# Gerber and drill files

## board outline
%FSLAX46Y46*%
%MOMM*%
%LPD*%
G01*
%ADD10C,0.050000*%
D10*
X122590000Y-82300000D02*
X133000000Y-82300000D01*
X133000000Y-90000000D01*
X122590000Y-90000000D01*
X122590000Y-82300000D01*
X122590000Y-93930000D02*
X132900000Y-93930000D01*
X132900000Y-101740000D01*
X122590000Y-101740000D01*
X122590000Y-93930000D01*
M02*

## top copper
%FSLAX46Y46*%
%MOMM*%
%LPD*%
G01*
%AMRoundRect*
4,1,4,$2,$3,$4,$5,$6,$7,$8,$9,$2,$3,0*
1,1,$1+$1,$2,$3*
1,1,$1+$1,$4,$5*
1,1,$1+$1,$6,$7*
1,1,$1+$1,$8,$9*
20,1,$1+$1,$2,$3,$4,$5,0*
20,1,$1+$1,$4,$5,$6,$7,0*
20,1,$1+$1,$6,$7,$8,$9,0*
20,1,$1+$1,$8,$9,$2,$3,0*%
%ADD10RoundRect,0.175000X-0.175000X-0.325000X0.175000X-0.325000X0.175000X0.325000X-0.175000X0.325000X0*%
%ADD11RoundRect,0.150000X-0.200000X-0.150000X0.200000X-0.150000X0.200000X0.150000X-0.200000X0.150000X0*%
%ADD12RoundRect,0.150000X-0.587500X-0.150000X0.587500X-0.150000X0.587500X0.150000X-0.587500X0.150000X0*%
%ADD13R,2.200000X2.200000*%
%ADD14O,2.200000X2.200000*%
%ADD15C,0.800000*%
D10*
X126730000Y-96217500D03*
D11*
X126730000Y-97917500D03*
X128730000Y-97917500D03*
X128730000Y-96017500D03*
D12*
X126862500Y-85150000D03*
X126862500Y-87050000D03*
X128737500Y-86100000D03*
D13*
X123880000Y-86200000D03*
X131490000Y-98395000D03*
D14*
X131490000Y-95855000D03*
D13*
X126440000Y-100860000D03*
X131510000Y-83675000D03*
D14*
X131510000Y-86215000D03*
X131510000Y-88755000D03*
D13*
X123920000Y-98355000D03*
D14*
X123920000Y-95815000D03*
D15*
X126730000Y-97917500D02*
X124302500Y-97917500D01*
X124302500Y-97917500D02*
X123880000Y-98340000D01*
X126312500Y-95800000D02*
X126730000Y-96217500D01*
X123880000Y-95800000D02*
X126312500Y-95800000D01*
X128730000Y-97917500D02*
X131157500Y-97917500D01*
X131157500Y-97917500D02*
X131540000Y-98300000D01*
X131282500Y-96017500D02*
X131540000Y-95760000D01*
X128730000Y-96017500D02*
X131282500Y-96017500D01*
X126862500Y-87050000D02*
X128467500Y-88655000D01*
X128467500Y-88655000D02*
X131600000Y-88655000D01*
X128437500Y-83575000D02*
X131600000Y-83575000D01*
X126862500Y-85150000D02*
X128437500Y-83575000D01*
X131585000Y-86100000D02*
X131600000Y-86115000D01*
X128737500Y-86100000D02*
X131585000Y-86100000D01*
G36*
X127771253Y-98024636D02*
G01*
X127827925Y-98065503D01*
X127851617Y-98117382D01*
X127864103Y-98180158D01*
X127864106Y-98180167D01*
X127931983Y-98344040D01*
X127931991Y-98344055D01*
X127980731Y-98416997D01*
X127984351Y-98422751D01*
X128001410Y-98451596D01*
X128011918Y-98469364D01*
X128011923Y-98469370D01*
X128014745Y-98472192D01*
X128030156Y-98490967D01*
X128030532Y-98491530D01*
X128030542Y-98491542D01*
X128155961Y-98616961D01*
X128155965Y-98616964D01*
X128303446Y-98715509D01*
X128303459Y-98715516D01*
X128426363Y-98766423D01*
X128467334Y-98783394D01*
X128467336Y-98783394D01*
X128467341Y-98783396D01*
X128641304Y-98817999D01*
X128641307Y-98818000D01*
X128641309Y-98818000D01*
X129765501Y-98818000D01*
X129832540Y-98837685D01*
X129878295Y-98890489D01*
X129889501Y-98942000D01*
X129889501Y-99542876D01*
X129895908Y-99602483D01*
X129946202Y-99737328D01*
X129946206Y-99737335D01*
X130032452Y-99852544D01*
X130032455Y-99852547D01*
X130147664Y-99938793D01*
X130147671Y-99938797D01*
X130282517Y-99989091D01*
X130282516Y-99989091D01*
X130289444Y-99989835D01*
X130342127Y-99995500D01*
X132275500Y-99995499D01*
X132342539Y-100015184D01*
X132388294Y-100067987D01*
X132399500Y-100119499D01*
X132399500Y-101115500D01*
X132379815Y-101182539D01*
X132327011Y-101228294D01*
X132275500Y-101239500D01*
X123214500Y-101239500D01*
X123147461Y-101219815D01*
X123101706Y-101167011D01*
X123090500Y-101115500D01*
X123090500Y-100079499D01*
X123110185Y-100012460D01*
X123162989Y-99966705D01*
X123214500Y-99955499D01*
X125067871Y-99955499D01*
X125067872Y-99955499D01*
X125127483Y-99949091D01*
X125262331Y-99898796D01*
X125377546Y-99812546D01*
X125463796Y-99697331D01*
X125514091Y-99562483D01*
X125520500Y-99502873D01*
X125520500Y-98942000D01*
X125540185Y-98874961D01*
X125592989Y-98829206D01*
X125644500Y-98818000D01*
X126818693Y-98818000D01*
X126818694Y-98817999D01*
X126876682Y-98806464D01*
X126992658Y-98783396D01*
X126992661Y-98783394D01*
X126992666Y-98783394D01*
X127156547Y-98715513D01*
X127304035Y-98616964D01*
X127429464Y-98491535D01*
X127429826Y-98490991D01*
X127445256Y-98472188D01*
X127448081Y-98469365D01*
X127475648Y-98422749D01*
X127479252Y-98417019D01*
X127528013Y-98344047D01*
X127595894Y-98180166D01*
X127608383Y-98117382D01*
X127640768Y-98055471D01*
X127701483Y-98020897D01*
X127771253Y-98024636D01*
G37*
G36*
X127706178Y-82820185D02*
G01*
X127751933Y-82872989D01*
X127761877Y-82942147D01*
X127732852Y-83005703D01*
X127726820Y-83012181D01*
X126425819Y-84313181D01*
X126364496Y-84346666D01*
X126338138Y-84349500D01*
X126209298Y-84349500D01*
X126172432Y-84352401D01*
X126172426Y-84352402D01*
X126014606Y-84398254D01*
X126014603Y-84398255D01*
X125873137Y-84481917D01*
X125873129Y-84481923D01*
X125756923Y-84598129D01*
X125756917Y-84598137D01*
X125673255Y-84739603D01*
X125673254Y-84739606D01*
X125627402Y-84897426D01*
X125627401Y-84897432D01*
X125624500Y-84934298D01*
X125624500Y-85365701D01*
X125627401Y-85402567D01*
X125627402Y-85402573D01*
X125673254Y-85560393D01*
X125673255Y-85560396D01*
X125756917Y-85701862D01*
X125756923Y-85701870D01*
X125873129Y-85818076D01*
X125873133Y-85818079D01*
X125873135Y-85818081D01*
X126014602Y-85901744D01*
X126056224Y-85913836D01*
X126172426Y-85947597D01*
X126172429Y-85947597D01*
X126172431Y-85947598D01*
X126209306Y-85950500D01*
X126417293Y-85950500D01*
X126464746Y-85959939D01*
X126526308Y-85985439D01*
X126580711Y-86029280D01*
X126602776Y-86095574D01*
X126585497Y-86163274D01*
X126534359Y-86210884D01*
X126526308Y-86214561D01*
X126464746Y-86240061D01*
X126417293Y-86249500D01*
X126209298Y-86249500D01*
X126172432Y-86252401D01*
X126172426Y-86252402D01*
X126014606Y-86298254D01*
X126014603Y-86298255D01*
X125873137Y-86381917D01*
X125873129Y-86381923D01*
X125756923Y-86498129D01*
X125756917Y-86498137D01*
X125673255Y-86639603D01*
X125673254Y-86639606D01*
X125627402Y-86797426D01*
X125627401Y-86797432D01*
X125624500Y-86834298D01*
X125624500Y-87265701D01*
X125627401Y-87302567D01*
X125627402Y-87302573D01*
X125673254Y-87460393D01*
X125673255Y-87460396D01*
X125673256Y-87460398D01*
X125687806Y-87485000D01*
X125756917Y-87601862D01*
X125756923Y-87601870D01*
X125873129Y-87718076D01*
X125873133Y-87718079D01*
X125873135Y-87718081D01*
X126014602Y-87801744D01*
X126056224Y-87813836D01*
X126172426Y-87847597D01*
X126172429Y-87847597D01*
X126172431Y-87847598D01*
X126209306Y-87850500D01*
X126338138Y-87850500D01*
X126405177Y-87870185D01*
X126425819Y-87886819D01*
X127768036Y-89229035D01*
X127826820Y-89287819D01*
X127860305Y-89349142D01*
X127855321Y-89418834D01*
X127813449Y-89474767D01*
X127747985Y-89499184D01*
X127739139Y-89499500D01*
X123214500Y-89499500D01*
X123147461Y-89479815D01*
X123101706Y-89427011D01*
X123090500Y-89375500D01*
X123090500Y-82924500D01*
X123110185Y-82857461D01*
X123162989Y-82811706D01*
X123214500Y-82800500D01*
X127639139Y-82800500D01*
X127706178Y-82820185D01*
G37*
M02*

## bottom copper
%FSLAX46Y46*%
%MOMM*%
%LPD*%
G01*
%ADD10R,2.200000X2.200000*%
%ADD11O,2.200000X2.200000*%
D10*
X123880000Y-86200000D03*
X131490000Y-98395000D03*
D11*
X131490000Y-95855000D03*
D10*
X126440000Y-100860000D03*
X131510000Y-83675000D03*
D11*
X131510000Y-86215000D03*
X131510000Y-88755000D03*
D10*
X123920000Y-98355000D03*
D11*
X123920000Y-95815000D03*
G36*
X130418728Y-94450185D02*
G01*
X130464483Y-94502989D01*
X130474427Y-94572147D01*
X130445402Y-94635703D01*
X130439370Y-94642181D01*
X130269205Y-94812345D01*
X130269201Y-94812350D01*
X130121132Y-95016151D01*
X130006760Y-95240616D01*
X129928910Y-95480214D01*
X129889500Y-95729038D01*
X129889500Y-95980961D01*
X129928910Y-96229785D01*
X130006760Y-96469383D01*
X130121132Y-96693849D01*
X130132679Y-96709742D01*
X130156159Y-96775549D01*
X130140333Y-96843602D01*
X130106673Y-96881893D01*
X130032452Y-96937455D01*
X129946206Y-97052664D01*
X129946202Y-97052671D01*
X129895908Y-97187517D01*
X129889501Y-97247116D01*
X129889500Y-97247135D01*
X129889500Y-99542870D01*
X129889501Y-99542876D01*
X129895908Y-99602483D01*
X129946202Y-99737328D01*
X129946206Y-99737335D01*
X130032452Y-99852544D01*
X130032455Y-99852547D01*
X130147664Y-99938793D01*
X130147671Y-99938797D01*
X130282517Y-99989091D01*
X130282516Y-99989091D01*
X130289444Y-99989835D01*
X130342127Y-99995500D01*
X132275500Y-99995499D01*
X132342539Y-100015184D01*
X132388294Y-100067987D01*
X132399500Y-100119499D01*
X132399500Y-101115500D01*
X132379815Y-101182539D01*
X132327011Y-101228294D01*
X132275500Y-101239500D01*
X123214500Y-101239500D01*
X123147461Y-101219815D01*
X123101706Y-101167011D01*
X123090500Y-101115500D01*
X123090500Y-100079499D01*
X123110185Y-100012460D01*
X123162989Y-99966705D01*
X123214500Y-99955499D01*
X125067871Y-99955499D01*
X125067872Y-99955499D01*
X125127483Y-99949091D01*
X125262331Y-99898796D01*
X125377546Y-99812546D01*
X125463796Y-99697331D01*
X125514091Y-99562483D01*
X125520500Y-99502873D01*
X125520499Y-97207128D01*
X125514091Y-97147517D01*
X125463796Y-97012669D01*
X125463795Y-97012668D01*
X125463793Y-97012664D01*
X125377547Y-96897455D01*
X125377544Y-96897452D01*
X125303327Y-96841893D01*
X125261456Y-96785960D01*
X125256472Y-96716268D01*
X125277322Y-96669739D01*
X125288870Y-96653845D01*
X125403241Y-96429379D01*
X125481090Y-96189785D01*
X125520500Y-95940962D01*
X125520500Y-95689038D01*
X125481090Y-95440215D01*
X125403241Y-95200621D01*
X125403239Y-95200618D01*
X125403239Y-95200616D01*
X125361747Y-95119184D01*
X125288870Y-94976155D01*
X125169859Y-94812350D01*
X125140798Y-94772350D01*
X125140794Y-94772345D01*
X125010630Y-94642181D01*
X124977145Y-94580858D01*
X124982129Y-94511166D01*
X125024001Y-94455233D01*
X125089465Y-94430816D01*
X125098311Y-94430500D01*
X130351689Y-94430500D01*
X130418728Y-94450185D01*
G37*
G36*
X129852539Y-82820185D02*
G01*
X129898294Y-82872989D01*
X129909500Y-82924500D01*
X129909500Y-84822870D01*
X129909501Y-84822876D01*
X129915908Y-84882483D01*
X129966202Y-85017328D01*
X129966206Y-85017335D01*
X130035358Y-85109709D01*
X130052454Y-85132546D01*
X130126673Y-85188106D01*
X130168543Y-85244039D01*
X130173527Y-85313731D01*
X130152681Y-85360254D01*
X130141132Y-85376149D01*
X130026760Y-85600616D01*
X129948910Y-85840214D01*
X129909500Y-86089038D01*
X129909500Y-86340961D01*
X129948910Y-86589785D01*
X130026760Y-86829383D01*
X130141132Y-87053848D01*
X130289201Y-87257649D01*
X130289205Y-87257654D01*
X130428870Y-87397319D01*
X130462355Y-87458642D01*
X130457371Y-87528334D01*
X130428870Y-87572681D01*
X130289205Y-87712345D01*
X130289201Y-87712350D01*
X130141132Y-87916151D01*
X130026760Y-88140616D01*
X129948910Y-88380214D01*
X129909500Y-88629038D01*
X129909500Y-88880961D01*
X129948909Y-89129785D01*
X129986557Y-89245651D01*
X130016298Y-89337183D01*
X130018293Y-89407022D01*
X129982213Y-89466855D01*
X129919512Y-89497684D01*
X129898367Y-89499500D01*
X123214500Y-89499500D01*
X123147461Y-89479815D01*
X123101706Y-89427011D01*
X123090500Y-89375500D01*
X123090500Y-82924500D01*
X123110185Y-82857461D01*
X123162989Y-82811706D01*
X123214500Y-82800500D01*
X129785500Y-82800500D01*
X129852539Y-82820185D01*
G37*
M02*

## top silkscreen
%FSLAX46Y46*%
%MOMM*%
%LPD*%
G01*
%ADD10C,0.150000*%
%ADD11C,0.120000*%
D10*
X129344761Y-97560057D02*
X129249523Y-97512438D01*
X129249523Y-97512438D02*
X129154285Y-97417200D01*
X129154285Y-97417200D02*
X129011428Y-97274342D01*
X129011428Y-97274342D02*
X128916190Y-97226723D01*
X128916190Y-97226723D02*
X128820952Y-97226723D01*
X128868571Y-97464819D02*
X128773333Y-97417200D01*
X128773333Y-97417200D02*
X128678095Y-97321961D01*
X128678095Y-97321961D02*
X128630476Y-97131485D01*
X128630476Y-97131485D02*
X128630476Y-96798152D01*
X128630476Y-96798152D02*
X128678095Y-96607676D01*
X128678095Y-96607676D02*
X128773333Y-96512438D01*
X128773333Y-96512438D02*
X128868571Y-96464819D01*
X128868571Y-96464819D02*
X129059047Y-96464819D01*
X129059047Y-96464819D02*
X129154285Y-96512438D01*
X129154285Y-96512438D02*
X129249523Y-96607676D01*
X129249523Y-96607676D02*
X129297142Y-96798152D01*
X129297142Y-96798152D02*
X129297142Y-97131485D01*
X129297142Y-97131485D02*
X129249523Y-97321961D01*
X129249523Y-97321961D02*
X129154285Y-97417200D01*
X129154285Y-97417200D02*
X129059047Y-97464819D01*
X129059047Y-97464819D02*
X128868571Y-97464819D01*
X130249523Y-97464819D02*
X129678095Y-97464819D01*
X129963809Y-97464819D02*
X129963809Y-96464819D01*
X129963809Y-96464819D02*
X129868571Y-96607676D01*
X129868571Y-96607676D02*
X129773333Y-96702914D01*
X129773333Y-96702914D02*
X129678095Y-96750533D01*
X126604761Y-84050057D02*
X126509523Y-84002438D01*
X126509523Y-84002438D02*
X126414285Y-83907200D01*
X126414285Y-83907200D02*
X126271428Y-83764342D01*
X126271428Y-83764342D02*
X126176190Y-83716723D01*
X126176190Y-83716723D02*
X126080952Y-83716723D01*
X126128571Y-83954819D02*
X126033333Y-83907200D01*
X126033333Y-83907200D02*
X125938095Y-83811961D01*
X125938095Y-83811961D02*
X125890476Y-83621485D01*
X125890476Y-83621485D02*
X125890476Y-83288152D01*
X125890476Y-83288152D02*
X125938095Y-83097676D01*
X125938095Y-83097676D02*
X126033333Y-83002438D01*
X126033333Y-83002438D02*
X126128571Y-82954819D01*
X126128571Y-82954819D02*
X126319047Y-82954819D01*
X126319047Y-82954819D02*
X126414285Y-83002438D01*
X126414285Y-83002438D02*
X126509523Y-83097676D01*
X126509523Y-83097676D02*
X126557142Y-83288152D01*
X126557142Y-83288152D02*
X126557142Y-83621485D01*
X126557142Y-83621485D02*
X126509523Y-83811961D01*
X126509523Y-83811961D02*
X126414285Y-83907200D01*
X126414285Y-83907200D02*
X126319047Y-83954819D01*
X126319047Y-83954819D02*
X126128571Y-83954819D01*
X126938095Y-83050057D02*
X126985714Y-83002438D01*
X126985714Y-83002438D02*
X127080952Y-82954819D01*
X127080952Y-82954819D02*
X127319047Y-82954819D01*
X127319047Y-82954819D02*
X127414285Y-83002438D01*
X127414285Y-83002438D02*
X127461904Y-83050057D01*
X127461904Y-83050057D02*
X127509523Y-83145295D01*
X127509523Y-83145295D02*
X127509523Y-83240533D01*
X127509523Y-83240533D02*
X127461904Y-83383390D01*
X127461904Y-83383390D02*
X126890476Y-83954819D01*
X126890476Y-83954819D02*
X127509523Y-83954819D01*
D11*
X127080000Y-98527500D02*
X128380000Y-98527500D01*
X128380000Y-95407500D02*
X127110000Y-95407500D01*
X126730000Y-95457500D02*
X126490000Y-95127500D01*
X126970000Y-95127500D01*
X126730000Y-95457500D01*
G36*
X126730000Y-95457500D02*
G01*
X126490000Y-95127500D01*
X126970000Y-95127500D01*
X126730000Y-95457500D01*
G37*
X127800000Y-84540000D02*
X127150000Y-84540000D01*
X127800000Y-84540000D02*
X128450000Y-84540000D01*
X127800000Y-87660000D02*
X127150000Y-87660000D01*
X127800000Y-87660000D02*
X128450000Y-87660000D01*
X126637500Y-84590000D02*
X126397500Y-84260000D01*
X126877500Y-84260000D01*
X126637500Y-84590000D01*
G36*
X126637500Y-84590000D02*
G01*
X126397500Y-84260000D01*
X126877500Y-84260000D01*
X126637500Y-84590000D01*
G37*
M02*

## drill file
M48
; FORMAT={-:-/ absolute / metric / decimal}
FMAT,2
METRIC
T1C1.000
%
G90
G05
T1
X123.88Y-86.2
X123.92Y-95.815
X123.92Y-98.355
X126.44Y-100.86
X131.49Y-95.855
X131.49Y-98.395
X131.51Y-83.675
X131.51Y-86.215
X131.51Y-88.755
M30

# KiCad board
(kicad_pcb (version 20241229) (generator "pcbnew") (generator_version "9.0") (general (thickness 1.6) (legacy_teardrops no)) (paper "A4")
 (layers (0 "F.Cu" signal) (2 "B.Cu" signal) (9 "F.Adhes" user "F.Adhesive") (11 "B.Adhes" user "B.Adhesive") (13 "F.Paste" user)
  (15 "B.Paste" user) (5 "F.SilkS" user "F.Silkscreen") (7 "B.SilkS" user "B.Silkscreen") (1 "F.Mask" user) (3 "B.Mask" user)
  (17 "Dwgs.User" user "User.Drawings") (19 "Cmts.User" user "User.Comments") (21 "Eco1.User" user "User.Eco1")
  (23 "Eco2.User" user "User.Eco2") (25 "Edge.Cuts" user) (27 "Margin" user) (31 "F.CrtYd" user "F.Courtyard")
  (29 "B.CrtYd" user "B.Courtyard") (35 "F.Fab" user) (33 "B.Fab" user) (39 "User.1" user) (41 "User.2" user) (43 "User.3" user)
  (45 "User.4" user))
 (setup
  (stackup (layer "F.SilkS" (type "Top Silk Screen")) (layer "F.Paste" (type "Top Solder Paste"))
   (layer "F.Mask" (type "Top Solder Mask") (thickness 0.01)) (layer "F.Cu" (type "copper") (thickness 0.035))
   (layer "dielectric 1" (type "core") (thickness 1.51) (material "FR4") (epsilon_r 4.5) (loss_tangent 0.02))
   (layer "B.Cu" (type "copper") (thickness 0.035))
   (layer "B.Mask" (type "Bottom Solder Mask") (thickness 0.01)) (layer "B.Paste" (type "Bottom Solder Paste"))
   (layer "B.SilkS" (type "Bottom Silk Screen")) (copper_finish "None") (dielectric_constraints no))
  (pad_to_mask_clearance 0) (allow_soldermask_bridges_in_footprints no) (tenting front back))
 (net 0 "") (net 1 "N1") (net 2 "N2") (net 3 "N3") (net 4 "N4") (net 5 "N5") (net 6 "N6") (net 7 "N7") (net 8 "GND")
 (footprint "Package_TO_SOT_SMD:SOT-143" (layer "F.Cu") (at 127.73 96.9675)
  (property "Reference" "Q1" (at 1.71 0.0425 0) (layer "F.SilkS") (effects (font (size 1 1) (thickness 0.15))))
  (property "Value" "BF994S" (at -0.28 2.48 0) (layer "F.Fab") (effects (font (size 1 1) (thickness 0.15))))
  (fp_line (start -0.65 1.56) (end 0.65 1.56) (stroke (width 0.12) (type solid)) (layer "F.SilkS"))
  (fp_line (start 0.65 -1.56) (end -0.62 -1.56) (stroke (width 0.12) (type solid)) (layer "F.SilkS"))
  (fp_poly
   (pts (xy -1 -1.51) (xy -1.24 -1.84) (xy -0.76 -1.84) (xy -1 -1.51)) (stroke (width 0.12) (type solid)) (fill yes) (layer "F.SilkS"))
  (pad "1" smd roundrect (at -1 -0.75) (size 0.7 1) (layers "F.Cu" "F.Mask" "F.Paste") (roundrect_rratio 0.25) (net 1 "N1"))
  (pad "2" smd roundrect (at -1 0.95) (size 0.7 0.6) (layers "F.Cu" "F.Mask" "F.Paste") (roundrect_rratio 0.25) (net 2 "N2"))
  (pad "3" smd roundrect (at 1 0.95) (size 0.7 0.6) (layers "F.Cu" "F.Mask" "F.Paste") (roundrect_rratio 0.25) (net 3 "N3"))
  (pad "4" smd roundrect (at 1 -0.95) (size 0.7 0.6) (layers "F.Cu" "F.Mask" "F.Paste") (roundrect_rratio 0.25) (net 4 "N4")))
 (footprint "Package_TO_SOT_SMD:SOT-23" (layer "F.Cu") (at 127.8 86.1)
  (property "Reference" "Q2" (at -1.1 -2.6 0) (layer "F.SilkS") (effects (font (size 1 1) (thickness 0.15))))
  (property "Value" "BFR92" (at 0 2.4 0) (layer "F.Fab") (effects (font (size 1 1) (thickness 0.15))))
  (fp_line (start 0 -1.56) (end -0.65 -1.56) (stroke (width 0.12) (type solid)) (layer "F.SilkS"))
  (fp_line (start 0 -1.56) (end 0.65 -1.56) (stroke (width 0.12) (type solid)) (layer "F.SilkS"))
  (fp_line (start 0 1.56) (end -0.65 1.56) (stroke (width 0.12) (type solid)) (layer "F.SilkS"))
  (fp_line (start 0 1.56) (end 0.65 1.56) (stroke (width 0.12) (type solid)) (layer "F.SilkS"))
  (fp_poly
   (pts (xy -1.1625 -1.51) (xy -1.4025 -1.84) (xy -0.9225 -1.84) (xy -1.1625 -1.51)) (stroke (width 0.12) (type solid)) (fill yes)
   (layer "F.SilkS"))
  (pad "1" smd roundrect (at -0.9375 -0.95) (size 1.475 0.6) (layers "F.Cu" "F.Mask" "F.Paste") (roundrect_rratio 0.25) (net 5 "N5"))
  (pad "2" smd roundrect (at -0.9375 0.95) (size 1.475 0.6) (layers "F.Cu" "F.Mask" "F.Paste") (roundrect_rratio 0.25) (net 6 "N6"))
  (pad "3" smd roundrect (at 0.9375 0) (size 1.475 0.6) (layers "F.Cu" "F.Mask" "F.Paste") (roundrect_rratio 0.25) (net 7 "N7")))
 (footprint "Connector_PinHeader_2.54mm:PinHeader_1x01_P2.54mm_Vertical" (layer "B.Cu") (at 123.88 86.2)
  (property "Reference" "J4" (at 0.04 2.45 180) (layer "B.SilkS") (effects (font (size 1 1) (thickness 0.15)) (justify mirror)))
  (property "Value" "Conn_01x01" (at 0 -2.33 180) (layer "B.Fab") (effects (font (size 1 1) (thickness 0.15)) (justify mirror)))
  (pad "1" thru_hole rect (at 0 0) (size 2.2 2.2) (drill 1) (layers "*.Cu" "*.Mask") (remove_unused_layers no) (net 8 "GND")))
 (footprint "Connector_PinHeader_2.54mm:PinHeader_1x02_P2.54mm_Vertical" (layer "B.Cu") (at 131.49 98.395)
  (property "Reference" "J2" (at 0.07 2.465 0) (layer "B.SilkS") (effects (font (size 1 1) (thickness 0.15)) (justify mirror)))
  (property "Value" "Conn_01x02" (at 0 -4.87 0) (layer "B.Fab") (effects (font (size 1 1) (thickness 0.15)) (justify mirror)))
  (pad "1" thru_hole rect (at 0 0) (size 2.2 2.2) (drill 1) (layers "*.Cu" "*.Mask") (remove_unused_layers no) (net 3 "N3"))
  (pad "2" thru_hole oval (at 0 -2.54) (size 2.2 2.2) (drill 1) (layers "*.Cu" "*.Mask") (remove_unused_layers no) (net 4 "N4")))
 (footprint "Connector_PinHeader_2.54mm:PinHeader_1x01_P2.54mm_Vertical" (layer "B.Cu") (at 126.44 100.86)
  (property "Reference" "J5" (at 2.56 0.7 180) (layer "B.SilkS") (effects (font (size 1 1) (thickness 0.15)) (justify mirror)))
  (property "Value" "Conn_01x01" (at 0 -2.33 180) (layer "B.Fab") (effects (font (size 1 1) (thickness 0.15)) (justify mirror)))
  (pad "1" thru_hole rect (at 0 0) (size 2.2 2.2) (drill 1) (layers "*.Cu" "*.Mask") (remove_unused_layers no) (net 8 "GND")))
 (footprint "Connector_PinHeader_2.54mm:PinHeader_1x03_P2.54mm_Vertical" (layer "B.Cu") (at 131.51 83.675 180)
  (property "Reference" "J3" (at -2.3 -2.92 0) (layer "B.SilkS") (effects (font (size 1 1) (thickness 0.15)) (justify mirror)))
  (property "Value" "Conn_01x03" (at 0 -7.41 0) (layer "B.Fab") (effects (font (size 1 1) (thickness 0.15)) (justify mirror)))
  (pad "1" thru_hole rect (at 0 0 180) (size 2.2 2.2) (drill 1) (layers "*.Cu" "*.Mask") (remove_unused_layers no) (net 5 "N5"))
  (pad "2" thru_hole oval (at 0 -2.54 180) (size 2.2 2.2) (drill 1) (layers "*.Cu" "*.Mask") (remove_unused_layers no) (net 7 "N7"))
  (pad "3" thru_hole oval (at 0 -5.08 180) (size 2.2 2.2) (drill 1) (layers "*.Cu" "*.Mask") (remove_unused_layers no) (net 6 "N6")))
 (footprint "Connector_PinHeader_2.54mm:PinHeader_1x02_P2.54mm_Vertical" (layer "B.Cu") (at 123.92 98.355)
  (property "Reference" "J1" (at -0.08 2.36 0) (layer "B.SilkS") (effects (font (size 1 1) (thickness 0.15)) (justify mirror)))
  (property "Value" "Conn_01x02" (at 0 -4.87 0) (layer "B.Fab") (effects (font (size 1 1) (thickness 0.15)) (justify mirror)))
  (pad "1" thru_hole rect (at 0 0) (size 2.2 2.2) (drill 1) (layers "*.Cu" "*.Mask") (remove_unused_layers no) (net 2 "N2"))
  (pad "2" thru_hole oval (at 0 -2.54) (size 2.2 2.2) (drill 1) (layers "*.Cu" "*.Mask") (remove_unused_layers no) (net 1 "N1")))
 (gr_rect (start 122.59 82.3) (end 133 90) (stroke (width 0.05) (type default)) (fill no) (layer "Edge.Cuts"))
 (gr_rect (start 122.59 93.93) (end 132.9 101.74) (stroke (width 0.05) (type default)) (fill no) (layer "Edge.Cuts"))
 (segment (start 126.73 97.9175) (end 124.3025 97.9175) (width 0.8) (layer "F.Cu") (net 2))
 (segment (start 124.3025 97.9175) (end 123.88 98.34) (width 0.8) (layer "F.Cu") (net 2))
 (segment (start 126.3125 95.8) (end 126.73 96.2175) (width 0.8) (layer "F.Cu") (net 1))
 (segment (start 123.88 95.8) (end 126.3125 95.8) (width 0.8) (layer "F.Cu") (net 1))
 (segment (start 128.73 97.9175) (end 131.1575 97.9175) (width 0.8) (layer "F.Cu") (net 3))
 (segment (start 131.1575 97.9175) (end 131.54 98.3) (width 0.8) (layer "F.Cu") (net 3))
 (segment (start 131.2825 96.0175) (end 131.54 95.76) (width 0.8) (layer "F.Cu") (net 4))
 (segment (start 128.73 96.0175) (end 131.2825 96.0175) (width 0.8) (layer "F.Cu") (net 4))
 (segment (start 126.8625 87.05) (end 128.4675 88.655) (width 0.8) (layer "F.Cu") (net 6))
 (segment (start 128.4675 88.655) (end 131.6 88.655) (width 0.8) (layer "F.Cu") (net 6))
 (segment (start 128.4375 83.575) (end 131.6 83.575) (width 0.8) (layer "F.Cu") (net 5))
 (segment (start 126.8625 85.15) (end 128.4375 83.575) (width 0.8) (layer "F.Cu") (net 5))
 (segment (start 131.585 86.1) (end 131.6 86.115) (width 0.8) (layer "F.Cu") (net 7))
 (segment (start 128.7375 86.1) (end 131.585 86.1) (width 0.8) (layer "F.Cu") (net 7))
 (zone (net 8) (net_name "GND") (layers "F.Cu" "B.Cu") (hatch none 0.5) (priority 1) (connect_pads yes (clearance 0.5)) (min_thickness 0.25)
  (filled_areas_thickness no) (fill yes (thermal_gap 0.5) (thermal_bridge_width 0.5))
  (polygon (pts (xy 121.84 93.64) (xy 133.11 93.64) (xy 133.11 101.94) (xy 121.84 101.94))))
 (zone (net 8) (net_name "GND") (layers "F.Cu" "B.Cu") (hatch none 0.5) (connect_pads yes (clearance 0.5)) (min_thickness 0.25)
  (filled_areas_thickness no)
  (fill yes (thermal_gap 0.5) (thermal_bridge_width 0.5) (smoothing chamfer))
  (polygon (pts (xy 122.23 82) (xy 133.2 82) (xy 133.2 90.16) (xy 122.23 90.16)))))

